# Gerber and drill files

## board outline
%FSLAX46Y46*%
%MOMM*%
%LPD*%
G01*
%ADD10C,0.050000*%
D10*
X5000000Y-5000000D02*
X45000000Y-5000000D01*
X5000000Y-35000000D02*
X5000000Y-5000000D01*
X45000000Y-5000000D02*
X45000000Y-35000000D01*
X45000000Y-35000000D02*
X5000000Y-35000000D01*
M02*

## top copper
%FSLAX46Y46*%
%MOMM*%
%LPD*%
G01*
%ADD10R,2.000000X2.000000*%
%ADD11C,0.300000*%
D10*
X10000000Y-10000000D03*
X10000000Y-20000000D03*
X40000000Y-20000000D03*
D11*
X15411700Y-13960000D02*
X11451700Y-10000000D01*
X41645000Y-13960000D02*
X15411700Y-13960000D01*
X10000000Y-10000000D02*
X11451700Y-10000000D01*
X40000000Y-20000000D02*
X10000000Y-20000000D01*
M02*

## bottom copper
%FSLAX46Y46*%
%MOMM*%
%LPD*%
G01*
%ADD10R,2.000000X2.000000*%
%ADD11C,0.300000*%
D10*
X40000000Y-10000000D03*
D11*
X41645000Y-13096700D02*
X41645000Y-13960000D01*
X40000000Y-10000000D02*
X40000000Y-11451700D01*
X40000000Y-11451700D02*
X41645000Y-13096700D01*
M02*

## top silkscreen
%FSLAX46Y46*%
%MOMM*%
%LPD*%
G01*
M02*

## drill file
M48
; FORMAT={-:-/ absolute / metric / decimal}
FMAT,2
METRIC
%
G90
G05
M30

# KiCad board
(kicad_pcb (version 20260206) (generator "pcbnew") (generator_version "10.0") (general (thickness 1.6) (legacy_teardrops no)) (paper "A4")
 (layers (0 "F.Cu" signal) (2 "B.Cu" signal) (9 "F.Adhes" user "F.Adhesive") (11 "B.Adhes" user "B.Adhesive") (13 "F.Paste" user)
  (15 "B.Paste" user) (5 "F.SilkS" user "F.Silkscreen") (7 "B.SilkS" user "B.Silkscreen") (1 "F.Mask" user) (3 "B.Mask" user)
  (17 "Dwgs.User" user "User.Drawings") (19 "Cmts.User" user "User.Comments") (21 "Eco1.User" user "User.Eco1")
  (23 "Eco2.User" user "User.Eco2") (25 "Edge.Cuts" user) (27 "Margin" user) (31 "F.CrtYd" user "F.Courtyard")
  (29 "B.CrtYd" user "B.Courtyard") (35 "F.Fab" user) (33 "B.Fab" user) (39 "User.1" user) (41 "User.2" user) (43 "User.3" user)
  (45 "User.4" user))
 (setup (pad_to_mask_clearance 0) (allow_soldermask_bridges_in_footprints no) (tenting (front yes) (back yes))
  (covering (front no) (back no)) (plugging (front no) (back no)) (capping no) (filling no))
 (gr_line (start 5 5) (end 45 5) (stroke (width 0.05) (type default)) (layer "Edge.Cuts"))
 (gr_line (start 5 35) (end 5 5) (stroke (width 0.05) (type default)) (layer "Edge.Cuts"))
 (gr_line (start 45 5) (end 45 35) (stroke (width 0.05) (type default)) (layer "Edge.Cuts"))
 (gr_line (start 45 35) (end 5 35) (stroke (width 0.05) (type default)) (layer "Edge.Cuts"))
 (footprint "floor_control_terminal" (layer "F.Cu") (at 10 10)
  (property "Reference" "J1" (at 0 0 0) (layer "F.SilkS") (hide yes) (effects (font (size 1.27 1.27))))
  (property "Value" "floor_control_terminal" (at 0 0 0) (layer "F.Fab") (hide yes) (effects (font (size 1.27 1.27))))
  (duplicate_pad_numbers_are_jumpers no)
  (pad "1" smd rect (at 0 0) (size 2 2) (layers "F.Cu" "F.Paste" "F.Mask") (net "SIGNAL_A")))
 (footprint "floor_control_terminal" (layer "B.Cu") (at 40 10)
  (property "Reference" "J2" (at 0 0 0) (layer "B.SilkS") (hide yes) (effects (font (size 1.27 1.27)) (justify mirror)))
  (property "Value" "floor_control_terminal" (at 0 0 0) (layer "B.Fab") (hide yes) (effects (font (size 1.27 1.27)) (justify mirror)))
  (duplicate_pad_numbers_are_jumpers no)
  (pad "1" smd rect (at 0 0) (size 2 2) (layers "B.Cu" "B.Paste" "B.Mask") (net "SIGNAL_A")))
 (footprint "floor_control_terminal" (layer "F.Cu") (at 10 20)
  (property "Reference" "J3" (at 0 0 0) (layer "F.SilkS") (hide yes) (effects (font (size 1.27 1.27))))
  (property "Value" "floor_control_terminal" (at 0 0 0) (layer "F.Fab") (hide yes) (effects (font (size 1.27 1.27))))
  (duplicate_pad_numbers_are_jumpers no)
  (pad "1" smd rect (at 0 0) (size 2 2) (layers "F.Cu" "F.Paste" "F.Mask") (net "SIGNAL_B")))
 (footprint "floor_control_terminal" (layer "F.Cu") (at 40 20)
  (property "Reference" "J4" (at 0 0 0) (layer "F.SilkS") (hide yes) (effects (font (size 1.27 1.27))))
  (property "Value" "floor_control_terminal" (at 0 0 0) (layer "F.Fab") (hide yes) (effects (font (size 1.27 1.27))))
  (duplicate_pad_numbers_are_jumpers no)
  (pad "1" smd rect (at 0 0) (size 2 2) (layers "F.Cu" "F.Paste" "F.Mask") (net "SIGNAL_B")))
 (segment (start 15.4117 13.96) (end 11.4517 10) (width 0.3) (layer "F.Cu") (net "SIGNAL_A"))
 (segment (start 41.645 13.96) (end 15.4117 13.96) (width 0.3) (layer "F.Cu") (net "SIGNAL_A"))
 (segment (start 10 10) (end 11.4517 10) (width 0.3) (layer "F.Cu") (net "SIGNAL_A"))
 (segment (start 41.645 13.0967) (end 41.645 13.96) (width 0.3) (layer "B.Cu") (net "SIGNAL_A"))
 (segment (start 40 10) (end 40 11.4517) (width 0.3) (layer "B.Cu") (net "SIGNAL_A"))
 (segment (start 40 11.4517) (end 41.645 13.0967) (width 0.3) (layer "B.Cu") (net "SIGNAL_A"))
 (segment (start 40 20) (end 10 20) (width 0.3) (layer "F.Cu") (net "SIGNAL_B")))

